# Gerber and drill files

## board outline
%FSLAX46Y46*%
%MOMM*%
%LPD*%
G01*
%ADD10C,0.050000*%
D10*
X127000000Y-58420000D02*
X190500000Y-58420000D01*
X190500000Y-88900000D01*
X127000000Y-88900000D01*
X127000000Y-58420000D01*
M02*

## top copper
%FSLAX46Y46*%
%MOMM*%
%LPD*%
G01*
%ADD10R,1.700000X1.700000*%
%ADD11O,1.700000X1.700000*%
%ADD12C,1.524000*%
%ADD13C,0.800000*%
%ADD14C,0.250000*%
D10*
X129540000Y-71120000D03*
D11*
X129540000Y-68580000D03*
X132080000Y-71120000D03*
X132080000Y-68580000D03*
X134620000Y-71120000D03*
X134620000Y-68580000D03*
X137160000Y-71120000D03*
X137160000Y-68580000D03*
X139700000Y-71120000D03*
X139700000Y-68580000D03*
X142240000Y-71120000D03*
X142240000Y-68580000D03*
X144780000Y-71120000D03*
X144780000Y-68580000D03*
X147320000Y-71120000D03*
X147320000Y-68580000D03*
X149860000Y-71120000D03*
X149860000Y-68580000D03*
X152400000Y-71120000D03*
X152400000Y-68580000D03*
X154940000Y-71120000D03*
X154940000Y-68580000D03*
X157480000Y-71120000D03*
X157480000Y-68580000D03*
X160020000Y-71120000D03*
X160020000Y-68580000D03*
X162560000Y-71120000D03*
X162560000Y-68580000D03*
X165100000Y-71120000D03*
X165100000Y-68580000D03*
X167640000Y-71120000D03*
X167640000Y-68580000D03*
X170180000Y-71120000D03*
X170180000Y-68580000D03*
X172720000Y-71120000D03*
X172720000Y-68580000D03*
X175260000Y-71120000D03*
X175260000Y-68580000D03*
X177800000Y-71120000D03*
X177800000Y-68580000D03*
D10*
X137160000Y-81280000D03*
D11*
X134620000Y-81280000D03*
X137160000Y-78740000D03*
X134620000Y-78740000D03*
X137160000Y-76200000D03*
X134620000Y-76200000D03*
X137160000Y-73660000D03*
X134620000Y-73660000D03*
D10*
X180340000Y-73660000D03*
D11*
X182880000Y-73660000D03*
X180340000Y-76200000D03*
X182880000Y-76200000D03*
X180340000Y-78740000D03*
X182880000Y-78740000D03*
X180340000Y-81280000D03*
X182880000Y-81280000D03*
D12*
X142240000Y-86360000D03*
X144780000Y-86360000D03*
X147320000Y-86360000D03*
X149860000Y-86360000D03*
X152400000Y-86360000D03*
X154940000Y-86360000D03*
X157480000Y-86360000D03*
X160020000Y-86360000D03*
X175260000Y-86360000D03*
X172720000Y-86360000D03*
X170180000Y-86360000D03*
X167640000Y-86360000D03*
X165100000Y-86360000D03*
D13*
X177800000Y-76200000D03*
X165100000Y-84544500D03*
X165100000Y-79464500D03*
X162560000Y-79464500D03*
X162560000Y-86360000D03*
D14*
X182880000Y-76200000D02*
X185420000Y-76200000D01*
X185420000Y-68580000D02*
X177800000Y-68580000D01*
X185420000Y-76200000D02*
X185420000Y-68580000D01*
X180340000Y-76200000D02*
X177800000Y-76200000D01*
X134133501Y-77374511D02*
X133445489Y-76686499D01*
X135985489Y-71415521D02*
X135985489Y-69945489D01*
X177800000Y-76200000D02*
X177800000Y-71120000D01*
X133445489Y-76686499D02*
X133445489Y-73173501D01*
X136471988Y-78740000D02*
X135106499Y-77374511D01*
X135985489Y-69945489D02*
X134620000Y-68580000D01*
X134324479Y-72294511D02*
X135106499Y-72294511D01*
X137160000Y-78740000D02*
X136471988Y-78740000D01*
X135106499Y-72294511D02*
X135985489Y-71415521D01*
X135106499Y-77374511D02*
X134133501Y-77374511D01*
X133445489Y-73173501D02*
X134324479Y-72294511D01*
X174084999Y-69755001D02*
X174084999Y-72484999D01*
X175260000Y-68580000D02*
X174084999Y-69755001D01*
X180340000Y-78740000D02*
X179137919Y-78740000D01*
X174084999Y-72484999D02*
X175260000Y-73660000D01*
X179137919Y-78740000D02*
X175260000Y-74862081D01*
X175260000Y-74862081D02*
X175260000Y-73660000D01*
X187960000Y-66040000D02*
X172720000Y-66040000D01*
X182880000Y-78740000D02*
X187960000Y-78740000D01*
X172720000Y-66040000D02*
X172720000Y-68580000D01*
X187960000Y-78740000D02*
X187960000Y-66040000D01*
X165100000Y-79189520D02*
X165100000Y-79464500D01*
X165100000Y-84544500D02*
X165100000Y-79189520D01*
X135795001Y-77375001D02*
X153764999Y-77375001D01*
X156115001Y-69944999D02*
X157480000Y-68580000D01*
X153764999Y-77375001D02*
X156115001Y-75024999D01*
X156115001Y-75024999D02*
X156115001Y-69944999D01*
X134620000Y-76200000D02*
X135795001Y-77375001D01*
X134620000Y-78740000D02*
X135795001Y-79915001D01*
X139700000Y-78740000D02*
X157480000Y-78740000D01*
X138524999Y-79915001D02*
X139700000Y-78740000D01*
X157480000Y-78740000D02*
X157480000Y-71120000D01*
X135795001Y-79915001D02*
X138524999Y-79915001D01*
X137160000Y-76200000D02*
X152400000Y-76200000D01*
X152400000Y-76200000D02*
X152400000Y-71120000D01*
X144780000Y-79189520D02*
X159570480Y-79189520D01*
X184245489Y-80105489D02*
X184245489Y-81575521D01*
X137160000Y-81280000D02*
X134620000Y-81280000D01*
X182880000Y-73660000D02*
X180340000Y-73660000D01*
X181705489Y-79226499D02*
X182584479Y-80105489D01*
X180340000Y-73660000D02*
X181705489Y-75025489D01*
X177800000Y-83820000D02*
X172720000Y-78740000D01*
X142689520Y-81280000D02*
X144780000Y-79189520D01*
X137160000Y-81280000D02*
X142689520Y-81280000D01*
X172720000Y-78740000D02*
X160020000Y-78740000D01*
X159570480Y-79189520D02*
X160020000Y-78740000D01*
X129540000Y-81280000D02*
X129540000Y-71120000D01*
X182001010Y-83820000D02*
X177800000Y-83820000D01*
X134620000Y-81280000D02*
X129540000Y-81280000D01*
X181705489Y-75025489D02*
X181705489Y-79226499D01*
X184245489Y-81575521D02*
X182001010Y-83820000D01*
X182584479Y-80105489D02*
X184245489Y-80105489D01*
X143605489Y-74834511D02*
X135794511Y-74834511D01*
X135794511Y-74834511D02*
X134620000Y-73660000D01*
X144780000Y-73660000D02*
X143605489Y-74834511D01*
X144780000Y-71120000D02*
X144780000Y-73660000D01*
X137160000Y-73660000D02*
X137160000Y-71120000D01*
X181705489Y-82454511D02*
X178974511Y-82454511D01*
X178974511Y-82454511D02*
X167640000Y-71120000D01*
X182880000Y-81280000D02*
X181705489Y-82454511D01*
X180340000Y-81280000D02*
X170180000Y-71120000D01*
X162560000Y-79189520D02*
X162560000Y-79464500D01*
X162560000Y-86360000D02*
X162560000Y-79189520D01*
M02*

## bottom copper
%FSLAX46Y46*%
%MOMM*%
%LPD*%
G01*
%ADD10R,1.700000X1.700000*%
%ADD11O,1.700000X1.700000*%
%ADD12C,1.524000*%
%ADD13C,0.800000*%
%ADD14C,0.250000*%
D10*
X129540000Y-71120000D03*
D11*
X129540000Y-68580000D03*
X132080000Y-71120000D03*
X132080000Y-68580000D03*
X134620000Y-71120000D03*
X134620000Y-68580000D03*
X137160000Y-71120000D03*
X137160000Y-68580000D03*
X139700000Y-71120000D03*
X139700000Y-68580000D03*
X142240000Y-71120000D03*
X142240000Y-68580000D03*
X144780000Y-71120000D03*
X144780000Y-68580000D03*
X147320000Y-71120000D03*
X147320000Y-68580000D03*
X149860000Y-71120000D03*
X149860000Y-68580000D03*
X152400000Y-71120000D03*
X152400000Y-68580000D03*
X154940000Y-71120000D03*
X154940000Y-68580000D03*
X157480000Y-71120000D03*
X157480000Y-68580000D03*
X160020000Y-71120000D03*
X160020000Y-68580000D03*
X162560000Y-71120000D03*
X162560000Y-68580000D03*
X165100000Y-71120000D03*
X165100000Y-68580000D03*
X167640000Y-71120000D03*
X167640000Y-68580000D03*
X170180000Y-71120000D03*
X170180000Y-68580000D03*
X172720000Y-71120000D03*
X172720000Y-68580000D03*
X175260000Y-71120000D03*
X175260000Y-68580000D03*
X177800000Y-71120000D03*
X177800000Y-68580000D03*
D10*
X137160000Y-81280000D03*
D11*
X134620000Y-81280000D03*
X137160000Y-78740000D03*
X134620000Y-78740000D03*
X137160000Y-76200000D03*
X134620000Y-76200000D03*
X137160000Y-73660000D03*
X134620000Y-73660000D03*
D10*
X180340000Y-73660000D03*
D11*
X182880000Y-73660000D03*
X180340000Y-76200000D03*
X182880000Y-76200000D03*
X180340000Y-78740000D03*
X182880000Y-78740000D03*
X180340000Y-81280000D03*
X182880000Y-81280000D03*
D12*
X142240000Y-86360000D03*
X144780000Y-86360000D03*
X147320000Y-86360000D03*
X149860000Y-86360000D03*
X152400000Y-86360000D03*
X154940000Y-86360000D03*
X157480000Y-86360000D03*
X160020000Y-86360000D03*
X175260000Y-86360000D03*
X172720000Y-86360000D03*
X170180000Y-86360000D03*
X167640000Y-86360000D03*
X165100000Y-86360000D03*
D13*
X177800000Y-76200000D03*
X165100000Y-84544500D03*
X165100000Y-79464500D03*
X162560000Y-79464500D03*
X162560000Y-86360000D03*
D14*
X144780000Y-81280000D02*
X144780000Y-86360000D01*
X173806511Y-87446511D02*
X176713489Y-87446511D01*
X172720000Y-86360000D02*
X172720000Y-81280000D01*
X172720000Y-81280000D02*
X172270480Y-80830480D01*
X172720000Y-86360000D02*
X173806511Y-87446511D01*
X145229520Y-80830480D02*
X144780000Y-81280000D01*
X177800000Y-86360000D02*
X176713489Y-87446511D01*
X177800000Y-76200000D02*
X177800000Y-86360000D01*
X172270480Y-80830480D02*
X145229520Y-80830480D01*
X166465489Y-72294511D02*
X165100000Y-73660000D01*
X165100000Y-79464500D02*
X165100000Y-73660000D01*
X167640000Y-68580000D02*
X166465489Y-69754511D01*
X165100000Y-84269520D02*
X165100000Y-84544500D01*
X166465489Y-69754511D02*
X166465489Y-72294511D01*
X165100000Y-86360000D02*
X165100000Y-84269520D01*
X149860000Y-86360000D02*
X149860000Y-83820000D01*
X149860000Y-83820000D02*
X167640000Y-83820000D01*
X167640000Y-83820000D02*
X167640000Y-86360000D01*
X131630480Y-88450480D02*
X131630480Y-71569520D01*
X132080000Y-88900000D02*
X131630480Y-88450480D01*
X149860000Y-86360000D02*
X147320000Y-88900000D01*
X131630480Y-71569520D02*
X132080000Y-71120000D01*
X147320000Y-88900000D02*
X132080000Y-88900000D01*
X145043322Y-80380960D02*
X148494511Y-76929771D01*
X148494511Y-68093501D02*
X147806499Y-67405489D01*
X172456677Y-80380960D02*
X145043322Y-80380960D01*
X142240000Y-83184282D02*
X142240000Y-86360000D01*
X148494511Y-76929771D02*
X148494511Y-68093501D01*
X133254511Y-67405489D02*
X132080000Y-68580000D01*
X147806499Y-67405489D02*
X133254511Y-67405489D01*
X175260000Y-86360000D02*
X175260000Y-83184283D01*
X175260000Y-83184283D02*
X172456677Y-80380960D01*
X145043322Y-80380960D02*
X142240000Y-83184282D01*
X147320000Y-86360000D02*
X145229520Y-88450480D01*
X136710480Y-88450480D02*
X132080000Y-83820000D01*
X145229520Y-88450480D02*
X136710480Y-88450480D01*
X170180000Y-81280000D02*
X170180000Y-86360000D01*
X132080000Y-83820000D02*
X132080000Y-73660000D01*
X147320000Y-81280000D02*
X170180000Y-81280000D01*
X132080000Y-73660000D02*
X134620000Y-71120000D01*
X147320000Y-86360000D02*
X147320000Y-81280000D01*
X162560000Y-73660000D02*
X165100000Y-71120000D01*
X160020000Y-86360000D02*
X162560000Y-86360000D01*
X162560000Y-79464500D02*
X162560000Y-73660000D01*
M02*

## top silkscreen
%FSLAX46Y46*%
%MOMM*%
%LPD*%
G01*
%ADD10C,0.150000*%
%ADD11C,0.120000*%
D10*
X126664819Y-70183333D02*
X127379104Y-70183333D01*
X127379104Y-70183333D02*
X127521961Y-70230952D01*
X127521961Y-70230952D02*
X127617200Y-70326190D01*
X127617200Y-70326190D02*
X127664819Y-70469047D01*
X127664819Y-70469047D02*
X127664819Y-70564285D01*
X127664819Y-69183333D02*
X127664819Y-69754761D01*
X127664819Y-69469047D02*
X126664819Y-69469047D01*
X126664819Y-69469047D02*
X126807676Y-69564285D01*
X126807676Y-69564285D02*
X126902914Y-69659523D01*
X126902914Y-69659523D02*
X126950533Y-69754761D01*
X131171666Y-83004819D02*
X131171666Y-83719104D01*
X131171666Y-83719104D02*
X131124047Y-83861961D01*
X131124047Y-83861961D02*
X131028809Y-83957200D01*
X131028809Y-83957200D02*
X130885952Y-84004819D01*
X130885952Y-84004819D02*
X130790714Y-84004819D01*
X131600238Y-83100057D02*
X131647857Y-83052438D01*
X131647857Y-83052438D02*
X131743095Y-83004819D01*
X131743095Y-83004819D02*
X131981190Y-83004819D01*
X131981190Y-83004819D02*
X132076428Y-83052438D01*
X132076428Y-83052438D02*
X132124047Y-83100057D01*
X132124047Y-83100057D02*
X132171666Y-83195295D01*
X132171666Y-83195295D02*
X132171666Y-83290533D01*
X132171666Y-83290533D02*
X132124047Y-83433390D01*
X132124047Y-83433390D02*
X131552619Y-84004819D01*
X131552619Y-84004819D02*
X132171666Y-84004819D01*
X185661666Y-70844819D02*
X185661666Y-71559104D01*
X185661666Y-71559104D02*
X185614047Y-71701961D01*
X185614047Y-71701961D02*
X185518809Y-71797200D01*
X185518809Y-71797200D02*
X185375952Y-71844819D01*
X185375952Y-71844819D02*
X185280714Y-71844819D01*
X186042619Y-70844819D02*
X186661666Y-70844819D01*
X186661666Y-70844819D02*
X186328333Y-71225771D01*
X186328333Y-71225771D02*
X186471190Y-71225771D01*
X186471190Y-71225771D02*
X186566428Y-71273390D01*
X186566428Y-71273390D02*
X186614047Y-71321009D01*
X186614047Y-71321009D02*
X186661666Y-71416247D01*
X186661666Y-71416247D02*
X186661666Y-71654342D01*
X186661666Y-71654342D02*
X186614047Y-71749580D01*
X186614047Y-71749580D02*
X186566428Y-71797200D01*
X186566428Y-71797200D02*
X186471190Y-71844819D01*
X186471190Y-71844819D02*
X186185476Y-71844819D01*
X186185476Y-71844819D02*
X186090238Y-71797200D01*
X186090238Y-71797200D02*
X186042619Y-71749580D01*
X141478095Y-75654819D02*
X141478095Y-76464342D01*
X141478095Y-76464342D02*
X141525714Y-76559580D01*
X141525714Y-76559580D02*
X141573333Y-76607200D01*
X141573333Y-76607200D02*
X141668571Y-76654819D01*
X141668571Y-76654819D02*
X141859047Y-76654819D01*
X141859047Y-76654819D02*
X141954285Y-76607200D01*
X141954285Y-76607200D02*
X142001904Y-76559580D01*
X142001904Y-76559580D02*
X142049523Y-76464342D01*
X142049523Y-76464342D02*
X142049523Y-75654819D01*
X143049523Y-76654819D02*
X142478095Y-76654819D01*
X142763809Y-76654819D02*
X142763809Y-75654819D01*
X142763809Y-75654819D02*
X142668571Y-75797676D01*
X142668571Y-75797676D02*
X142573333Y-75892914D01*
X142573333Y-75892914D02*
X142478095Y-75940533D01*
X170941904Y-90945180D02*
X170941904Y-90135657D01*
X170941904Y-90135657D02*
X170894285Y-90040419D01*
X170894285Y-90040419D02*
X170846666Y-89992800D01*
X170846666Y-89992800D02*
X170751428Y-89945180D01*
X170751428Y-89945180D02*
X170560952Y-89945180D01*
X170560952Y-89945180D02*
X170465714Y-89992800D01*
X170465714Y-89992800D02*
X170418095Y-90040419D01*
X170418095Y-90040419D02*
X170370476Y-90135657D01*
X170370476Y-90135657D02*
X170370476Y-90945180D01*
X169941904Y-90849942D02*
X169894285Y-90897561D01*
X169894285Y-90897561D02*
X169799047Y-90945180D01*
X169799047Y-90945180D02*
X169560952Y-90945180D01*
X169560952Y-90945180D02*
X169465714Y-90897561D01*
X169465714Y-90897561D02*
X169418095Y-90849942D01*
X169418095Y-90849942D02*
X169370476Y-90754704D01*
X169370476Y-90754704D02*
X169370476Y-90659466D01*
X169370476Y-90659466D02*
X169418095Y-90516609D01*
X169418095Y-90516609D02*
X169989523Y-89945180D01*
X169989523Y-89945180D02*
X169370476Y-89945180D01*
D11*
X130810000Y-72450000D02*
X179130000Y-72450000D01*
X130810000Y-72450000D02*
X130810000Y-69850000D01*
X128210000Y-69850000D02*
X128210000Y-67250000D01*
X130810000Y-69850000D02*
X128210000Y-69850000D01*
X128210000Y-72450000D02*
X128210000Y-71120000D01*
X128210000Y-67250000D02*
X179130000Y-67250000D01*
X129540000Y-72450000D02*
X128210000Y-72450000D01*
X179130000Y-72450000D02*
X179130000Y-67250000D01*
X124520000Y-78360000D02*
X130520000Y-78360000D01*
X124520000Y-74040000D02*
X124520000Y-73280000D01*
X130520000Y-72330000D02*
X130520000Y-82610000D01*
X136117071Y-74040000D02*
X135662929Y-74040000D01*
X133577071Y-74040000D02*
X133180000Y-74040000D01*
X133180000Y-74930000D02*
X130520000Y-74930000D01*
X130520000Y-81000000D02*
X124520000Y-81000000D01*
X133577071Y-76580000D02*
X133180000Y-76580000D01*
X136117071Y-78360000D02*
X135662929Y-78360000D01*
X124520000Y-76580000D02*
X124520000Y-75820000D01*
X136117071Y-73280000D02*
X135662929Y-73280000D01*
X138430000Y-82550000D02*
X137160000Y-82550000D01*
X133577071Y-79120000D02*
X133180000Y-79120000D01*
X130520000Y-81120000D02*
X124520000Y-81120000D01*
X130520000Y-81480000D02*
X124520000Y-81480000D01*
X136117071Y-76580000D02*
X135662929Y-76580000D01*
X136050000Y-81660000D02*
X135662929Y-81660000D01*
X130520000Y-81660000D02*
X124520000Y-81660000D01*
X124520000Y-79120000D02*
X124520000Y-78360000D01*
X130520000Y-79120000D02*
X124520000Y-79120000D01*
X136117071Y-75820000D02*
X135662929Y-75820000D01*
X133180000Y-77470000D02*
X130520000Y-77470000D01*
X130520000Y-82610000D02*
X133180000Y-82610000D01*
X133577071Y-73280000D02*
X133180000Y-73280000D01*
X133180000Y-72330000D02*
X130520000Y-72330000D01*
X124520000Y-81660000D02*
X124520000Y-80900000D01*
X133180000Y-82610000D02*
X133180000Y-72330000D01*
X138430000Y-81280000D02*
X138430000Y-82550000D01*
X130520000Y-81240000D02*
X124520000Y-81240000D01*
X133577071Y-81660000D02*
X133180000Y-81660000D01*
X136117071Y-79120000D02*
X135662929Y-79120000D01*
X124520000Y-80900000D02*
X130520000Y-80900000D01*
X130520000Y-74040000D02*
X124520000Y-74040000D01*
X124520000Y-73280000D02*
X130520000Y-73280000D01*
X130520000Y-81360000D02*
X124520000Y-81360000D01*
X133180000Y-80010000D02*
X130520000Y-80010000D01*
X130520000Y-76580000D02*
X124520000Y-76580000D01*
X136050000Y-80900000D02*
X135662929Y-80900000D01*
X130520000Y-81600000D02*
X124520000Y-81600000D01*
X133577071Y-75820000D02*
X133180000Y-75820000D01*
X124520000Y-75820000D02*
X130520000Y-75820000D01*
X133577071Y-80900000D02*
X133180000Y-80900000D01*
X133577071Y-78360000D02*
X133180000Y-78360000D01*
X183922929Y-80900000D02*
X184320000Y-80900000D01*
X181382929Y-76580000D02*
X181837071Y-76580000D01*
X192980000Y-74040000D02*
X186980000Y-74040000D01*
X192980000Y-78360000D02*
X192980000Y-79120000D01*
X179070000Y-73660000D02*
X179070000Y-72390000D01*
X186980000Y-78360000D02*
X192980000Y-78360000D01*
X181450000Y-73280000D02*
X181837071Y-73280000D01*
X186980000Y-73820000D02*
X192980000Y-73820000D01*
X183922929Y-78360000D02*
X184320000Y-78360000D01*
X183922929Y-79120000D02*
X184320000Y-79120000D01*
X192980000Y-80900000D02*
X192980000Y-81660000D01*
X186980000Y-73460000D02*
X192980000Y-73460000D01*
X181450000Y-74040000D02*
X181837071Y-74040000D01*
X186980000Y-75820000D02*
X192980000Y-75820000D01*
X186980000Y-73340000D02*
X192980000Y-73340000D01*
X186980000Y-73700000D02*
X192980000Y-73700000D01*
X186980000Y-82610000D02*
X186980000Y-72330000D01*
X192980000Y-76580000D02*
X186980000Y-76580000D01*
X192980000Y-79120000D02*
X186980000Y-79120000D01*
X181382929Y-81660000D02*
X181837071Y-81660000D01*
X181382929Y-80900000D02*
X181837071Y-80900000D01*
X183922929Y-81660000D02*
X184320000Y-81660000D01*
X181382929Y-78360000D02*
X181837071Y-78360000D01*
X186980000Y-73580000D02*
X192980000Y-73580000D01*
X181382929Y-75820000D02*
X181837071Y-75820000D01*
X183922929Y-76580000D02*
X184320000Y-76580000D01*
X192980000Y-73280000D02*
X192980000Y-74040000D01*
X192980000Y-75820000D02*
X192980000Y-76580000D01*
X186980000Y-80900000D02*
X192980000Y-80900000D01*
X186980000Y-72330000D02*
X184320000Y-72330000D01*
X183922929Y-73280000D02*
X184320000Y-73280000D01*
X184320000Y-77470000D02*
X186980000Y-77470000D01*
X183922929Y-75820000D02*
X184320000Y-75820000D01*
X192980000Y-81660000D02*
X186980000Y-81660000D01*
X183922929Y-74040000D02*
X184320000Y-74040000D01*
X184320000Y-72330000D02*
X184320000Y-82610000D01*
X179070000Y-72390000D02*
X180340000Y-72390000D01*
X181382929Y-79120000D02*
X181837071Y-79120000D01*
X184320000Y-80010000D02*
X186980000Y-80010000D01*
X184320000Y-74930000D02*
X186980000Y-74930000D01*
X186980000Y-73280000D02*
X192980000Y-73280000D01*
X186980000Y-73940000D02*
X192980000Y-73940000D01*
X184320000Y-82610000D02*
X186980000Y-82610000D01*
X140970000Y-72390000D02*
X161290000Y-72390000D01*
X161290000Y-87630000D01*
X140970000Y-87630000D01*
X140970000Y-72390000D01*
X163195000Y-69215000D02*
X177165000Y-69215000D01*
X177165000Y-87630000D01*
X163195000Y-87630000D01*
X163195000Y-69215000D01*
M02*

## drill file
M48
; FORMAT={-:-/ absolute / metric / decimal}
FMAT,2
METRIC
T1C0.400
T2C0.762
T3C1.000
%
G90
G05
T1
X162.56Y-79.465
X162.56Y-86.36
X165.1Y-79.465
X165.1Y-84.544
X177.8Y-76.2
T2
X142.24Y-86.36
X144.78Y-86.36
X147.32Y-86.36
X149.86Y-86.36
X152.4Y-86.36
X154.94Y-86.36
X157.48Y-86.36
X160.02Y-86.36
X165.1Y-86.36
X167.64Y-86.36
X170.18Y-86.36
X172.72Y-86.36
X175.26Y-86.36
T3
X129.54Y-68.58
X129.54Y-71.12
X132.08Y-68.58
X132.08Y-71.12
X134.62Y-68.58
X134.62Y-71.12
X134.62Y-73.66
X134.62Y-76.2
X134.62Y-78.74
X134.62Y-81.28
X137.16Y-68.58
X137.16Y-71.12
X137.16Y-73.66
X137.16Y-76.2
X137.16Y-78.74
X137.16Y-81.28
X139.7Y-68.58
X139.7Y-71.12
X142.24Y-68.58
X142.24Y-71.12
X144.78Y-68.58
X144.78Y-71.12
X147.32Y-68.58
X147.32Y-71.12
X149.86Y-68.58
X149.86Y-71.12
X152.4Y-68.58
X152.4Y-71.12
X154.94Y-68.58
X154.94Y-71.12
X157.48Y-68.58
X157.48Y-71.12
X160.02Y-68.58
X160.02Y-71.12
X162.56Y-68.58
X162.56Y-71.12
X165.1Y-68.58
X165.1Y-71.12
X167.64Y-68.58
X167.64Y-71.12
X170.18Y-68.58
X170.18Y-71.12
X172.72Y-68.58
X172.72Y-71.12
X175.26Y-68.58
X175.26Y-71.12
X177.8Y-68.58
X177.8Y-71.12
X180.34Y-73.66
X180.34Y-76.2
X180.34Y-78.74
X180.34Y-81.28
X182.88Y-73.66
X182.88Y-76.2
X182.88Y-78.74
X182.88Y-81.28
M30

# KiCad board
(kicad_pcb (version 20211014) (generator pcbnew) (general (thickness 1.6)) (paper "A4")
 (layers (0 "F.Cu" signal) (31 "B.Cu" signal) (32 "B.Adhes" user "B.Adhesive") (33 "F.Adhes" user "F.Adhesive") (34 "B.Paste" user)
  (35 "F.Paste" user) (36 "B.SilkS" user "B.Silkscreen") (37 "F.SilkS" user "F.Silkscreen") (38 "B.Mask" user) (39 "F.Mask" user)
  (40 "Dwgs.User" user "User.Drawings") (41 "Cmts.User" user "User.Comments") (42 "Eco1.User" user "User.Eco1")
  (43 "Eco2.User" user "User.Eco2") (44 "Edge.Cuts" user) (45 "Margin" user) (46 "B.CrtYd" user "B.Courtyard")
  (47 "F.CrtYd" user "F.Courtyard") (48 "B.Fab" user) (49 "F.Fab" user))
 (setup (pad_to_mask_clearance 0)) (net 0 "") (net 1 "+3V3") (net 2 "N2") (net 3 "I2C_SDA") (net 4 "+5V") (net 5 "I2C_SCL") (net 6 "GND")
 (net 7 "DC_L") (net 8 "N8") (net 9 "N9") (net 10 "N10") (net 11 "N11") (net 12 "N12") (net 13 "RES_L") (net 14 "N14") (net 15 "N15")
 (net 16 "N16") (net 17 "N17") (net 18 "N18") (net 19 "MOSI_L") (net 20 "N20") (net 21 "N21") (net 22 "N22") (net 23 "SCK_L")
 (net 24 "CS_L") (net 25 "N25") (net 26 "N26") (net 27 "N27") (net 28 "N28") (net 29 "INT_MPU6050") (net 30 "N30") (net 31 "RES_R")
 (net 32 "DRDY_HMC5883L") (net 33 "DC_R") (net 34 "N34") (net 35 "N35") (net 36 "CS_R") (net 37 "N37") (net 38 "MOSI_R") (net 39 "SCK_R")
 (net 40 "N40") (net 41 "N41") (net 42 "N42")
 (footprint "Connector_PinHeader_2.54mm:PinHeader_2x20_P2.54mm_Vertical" (layer "F.Cu") (at 129.54 71.12 90)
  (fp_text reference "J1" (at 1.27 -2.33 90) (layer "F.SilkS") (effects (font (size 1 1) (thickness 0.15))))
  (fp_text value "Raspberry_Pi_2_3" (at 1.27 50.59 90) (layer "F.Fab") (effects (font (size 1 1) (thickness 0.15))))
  (fp_line (start -1.33 1.27) (end -1.33 49.59) (layer "F.SilkS") (width 0.12))
  (fp_line (start -1.33 1.27) (end 1.27 1.27) (layer "F.SilkS") (width 0.12))
  (fp_line (start 1.27 -1.33) (end 3.87 -1.33) (layer "F.SilkS") (width 0.12))
  (fp_line (start 1.27 1.27) (end 1.27 -1.33) (layer "F.SilkS") (width 0.12))
  (fp_line (start -1.33 -1.33) (end 0 -1.33) (layer "F.SilkS") (width 0.12))
  (fp_line (start 3.87 -1.33) (end 3.87 49.59) (layer "F.SilkS") (width 0.12))
  (fp_line (start -1.33 0) (end -1.33 -1.33) (layer "F.SilkS") (width 0.12))
  (fp_line (start -1.33 49.59) (end 3.87 49.59) (layer "F.SilkS") (width 0.12))
  (pad "1" thru_hole rect locked (at 0 0 90) (size 1.7 1.7) (drill 1) (layers *.Cu *.Mask) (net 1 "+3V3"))
  (pad "2" thru_hole oval locked (at 2.54 0 90) (size 1.7 1.7) (drill 1) (layers *.Cu *.Mask) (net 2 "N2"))
  (pad "3" thru_hole oval locked (at 0 2.54 90) (size 1.7 1.7) (drill 1) (layers *.Cu *.Mask) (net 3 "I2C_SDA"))
  (pad "4" thru_hole oval locked (at 2.54 2.54 90) (size 1.7 1.7) (drill 1) (layers *.Cu *.Mask) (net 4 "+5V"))
  (pad "5" thru_hole oval locked (at 0 5.08 90) (size 1.7 1.7) (drill 1) (layers *.Cu *.Mask) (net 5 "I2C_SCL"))
  (pad "6" thru_hole oval locked (at 2.54 5.08 90) (size 1.7 1.7) (drill 1) (layers *.Cu *.Mask) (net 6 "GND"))
  (pad "7" thru_hole oval locked (at 0 7.62 90) (size 1.7 1.7) (drill 1) (layers *.Cu *.Mask) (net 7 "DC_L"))
  (pad "8" thru_hole oval locked (at 2.54 7.62 90) (size 1.7 1.7) (drill 1) (layers *.Cu *.Mask) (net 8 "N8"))
  (pad "9" thru_hole oval locked (at 0 10.16 90) (size 1.7 1.7) (drill 1) (layers *.Cu *.Mask) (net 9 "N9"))
  (pad "10" thru_hole oval locked (at 2.54 10.16 90) (size 1.7 1.7) (drill 1) (layers *.Cu *.Mask) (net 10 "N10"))
  (pad "11" thru_hole oval locked (at 0 12.7 90) (size 1.7 1.7) (drill 1) (layers *.Cu *.Mask) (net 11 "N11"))
  (pad "12" thru_hole oval locked (at 2.54 12.7 90) (size 1.7 1.7) (drill 1) (layers *.Cu *.Mask) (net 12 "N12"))
  (pad "13" thru_hole oval locked (at 0 15.24 90) (size 1.7 1.7) (drill 1) (layers *.Cu *.Mask) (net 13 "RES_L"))
  (pad "14" thru_hole oval locked (at 2.54 15.24 90) (size 1.7 1.7) (drill 1) (layers *.Cu *.Mask) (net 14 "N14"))
  (pad "15" thru_hole oval locked (at 0 17.78 90) (size 1.7 1.7) (drill 1) (layers *.Cu *.Mask) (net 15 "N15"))
  (pad "16" thru_hole oval locked (at 2.54 17.78 90) (size 1.7 1.7) (drill 1) (layers *.Cu *.Mask) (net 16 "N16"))
  (pad "17" thru_hole oval locked (at 0 20.32 90) (size 1.7 1.7) (drill 1) (layers *.Cu *.Mask) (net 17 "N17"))
  (pad "18" thru_hole oval locked (at 2.54 20.32 90) (size 1.7 1.7) (drill 1) (layers *.Cu *.Mask) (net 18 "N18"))
  (pad "19" thru_hole oval locked (at 0 22.86 90) (size 1.7 1.7) (drill 1) (layers *.Cu *.Mask) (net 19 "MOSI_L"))
  (pad "20" thru_hole oval locked (at 2.54 22.86 90) (size 1.7 1.7) (drill 1) (layers *.Cu *.Mask) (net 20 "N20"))
  (pad "21" thru_hole oval locked (at 0 25.4 90) (size 1.7 1.7) (drill 1) (layers *.Cu *.Mask) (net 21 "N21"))
  (pad "22" thru_hole oval locked (at 2.54 25.4 90) (size 1.7 1.7) (drill 1) (layers *.Cu *.Mask) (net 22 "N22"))
  (pad "23" thru_hole oval locked (at 0 27.94 90) (size 1.7 1.7) (drill 1) (layers *.Cu *.Mask) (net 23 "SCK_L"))
  (pad "24" thru_hole oval locked (at 2.54 27.94 90) (size 1.7 1.7) (drill 1) (layers *.Cu *.Mask) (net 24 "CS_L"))
  (pad "25" thru_hole oval locked (at 0 30.48 90) (size 1.7 1.7) (drill 1) (layers *.Cu *.Mask) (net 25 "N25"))
  (pad "26" thru_hole oval locked (at 2.54 30.48 90) (size 1.7 1.7) (drill 1) (layers *.Cu *.Mask) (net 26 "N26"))
  (pad "27" thru_hole oval locked (at 0 33.02 90) (size 1.7 1.7) (drill 1) (layers *.Cu *.Mask) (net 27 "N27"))
  (pad "28" thru_hole oval locked (at 2.54 33.02 90) (size 1.7 1.7) (drill 1) (layers *.Cu *.Mask) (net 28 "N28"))
  (pad "29" thru_hole oval locked (at 0 35.56 90) (size 1.7 1.7) (drill 1) (layers *.Cu *.Mask) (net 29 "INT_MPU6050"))
  (pad "30" thru_hole oval locked (at 2.54 35.56 90) (size 1.7 1.7) (drill 1) (layers *.Cu *.Mask) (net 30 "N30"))
  (pad "31" thru_hole oval locked (at 0 38.1 90) (size 1.7 1.7) (drill 1) (layers *.Cu *.Mask) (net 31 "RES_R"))
  (pad "32" thru_hole oval locked (at 2.54 38.1 90) (size 1.7 1.7) (drill 1) (layers *.Cu *.Mask) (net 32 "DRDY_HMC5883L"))
  (pad "33" thru_hole oval locked (at 0 40.64 90) (size 1.7 1.7) (drill 1) (layers *.Cu *.Mask) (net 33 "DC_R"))
  (pad "34" thru_hole oval locked (at 2.54 40.64 90) (size 1.7 1.7) (drill 1) (layers *.Cu *.Mask) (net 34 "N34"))
  (pad "35" thru_hole oval locked (at 0 43.18 90) (size 1.7 1.7) (drill 1) (layers *.Cu *.Mask) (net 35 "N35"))
  (pad "36" thru_hole oval locked (at 2.54 43.18 90) (size 1.7 1.7) (drill 1) (layers *.Cu *.Mask) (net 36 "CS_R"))
  (pad "37" thru_hole oval locked (at 0 45.72 90) (size 1.7 1.7) (drill 1) (layers *.Cu *.Mask) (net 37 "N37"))
  (pad "38" thru_hole oval locked (at 2.54 45.72 90) (size 1.7 1.7) (drill 1) (layers *.Cu *.Mask) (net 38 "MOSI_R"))
  (pad "39" thru_hole oval locked (at 0 48.26 90) (size 1.7 1.7) (drill 1) (layers *.Cu *.Mask) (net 6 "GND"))
  (pad "40" thru_hole oval locked (at 2.54 48.26 90) (size 1.7 1.7) (drill 1) (layers *.Cu *.Mask) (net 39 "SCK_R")))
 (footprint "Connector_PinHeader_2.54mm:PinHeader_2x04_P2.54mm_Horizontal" (layer "F.Cu") (at 137.16 81.28 180)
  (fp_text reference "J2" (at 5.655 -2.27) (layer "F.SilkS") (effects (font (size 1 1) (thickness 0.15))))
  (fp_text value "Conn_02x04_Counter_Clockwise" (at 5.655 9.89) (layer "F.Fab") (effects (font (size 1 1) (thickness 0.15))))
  (fp_line (start 12.64 2.92) (end 6.64 2.92) (layer "F.SilkS") (width 0.12))
  (fp_line (start 12.64 7.24) (end 12.64 8) (layer "F.SilkS") (width 0.12))
  (fp_line (start 6.64 8.95) (end 6.64 -1.33) (layer "F.SilkS") (width 0.12))
  (fp_line (start 1.042929 7.24) (end 1.497071 7.24) (layer "F.SilkS") (width 0.12))
  (fp_line (start 3.582929 7.24) (end 3.98 7.24) (layer "F.SilkS") (width 0.12))
  (fp_line (start 3.98 6.35) (end 6.64 6.35) (layer "F.SilkS") (width 0.12))
  (fp_line (start 6.64 0.28) (end 12.64 0.28) (layer "F.SilkS") (width 0.12))
  (fp_line (start 3.582929 4.7) (end 3.98 4.7) (layer "F.SilkS") (width 0.12))
  (fp_line (start 1.042929 2.92) (end 1.497071 2.92) (layer "F.SilkS") (width 0.12))
  (fp_line (start 12.64 4.7) (end 12.64 5.46) (layer "F.SilkS") (width 0.12))
  (fp_line (start 1.042929 8) (end 1.497071 8) (layer "F.SilkS") (width 0.12))
  (fp_line (start -1.27 -1.27) (end 0 -1.27) (layer "F.SilkS") (width 0.12))
  (fp_line (start 3.582929 2.16) (end 3.98 2.16) (layer "F.SilkS") (width 0.12))
  (fp_line (start 6.64 0.16) (end 12.64 0.16) (layer "F.SilkS") (width 0.12))
  (fp_line (start 6.64 -0.2) (end 12.64 -0.2) (layer "F.SilkS") (width 0.12))
  (fp_line (start 1.042929 4.7) (end 1.497071 4.7) (layer "F.SilkS") (width 0.12))
  (fp_line (start 1.11 -0.38) (end 1.497071 -0.38) (layer "F.SilkS") (width 0.12))
  (fp_line (start 6.64 -0.38) (end 12.64 -0.38) (layer "F.SilkS") (width 0.12))
  (fp_line (start 12.64 2.16) (end 12.64 2.92) (layer "F.SilkS") (width 0.12))
  (fp_line (start 6.64 2.16) (end 12.64 2.16) (layer "F.SilkS") (width 0.12))
  (fp_line (start 1.042929 5.46) (end 1.497071 5.46) (layer "F.SilkS") (width 0.12))
  (fp_line (start 3.98 3.81) (end 6.64 3.81) (layer "F.SilkS") (width 0.12))
  (fp_line (start 6.64 -1.33) (end 3.98 -1.33) (layer "F.SilkS") (width 0.12))
  (fp_line (start 3.582929 8) (end 3.98 8) (layer "F.SilkS") (width 0.12))
  (fp_line (start 3.98 8.95) (end 6.64 8.95) (layer "F.SilkS") (width 0.12))
  (fp_line (start 12.64 -0.38) (end 12.64 0.38) (layer "F.SilkS") (width 0.12))
  (fp_line (start 3.98 -1.33) (end 3.98 8.95) (layer "F.SilkS") (width 0.12))
  (fp_line (start -1.27 0) (end -1.27 -1.27) (layer "F.SilkS") (width 0.12))
  (fp_line (start 6.64 0.04) (end 12.64 0.04) (layer "F.SilkS") (width 0.12))
  (fp_line (start 3.582929 -0.38) (end 3.98 -0.38) (layer "F.SilkS") (width 0.12))
  (fp_line (start 1.042929 2.16) (end 1.497071 2.16) (layer "F.SilkS") (width 0.12))
  (fp_line (start 12.64 0.38) (end 6.64 0.38) (layer "F.SilkS") (width 0.12))
  (fp_line (start 6.64 7.24) (end 12.64 7.24) (layer "F.SilkS") (width 0.12))
  (fp_line (start 12.64 8) (end 6.64 8) (layer "F.SilkS") (width 0.12))
  (fp_line (start 6.64 -0.08) (end 12.64 -0.08) (layer "F.SilkS") (width 0.12))
  (fp_line (start 3.98 1.27) (end 6.64 1.27) (layer "F.SilkS") (width 0.12))
  (fp_line (start 6.64 4.7) (end 12.64 4.7) (layer "F.SilkS") (width 0.12))
  (fp_line (start 1.11 0.38) (end 1.497071 0.38) (layer "F.SilkS") (width 0.12))
  (fp_line (start 6.64 -0.32) (end 12.64 -0.32) (layer "F.SilkS") (width 0.12))
  (fp_line (start 3.582929 5.46) (end 3.98 5.46) (layer "F.SilkS") (width 0.12))
  (fp_line (start 12.64 5.46) (end 6.64 5.46) (layer "F.SilkS") (width 0.12))
  (fp_line (start 3.582929 0.38) (end 3.98 0.38) (layer "F.SilkS") (width 0.12))
  (fp_line (start 3.582929 2.92) (end 3.98 2.92) (layer "F.SilkS") (width 0.12))
  (pad "1" thru_hole rect locked (at 0 0 180) (size 1.7 1.7) (drill 1) (layers *.Cu *.Mask) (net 1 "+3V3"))
  (pad "2" thru_hole oval locked (at 2.54 0 180) (size 1.7 1.7) (drill 1) (layers *.Cu *.Mask) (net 1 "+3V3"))
  (pad "3" thru_hole oval locked (at 0 2.54 180) (size 1.7 1.7) (drill 1) (layers *.Cu *.Mask) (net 6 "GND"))
  (pad "4" thru_hole oval locked (at 2.54 2.54 180) (size 1.7 1.7) (drill 1) (layers *.Cu *.Mask) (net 23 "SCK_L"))
  (pad "5" thru_hole oval locked (at 0 5.08 180) (size 1.7 1.7) (drill 1) (layers *.Cu *.Mask) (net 19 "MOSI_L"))
  (pad "6" thru_hole oval locked (at 2.54 5.08 180) (size 1.7 1.7) (drill 1) (layers *.Cu *.Mask) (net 24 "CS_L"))
  (pad "7" thru_hole oval locked (at 0 7.62 180) (size 1.7 1.7) (drill 1) (layers *.Cu *.Mask) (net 7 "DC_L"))
  (pad "8" thru_hole oval locked (at 2.54 7.62 180) (size 1.7 1.7) (drill 1) (layers *.Cu *.Mask) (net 13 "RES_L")))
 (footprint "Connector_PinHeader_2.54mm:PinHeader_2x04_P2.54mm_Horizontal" (layer "F.Cu") (at 180.34 73.66)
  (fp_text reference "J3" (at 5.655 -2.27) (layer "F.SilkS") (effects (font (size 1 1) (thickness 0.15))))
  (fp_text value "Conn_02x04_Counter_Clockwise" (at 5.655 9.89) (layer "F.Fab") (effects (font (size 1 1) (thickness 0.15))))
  (fp_line (start 3.582929 7.24) (end 3.98 7.24) (layer "F.SilkS") (width 0.12))
  (fp_line (start 1.042929 2.92) (end 1.497071 2.92) (layer "F.SilkS") (width 0.12))
  (fp_line (start 12.64 0.38) (end 6.64 0.38) (layer "F.SilkS") (width 0.12))
  (fp_line (start 12.64 4.7) (end 12.64 5.46) (layer "F.SilkS") (width 0.12))
  (fp_line (start -1.27 0) (end -1.27 -1.27) (layer "F.SilkS") (width 0.12))
  (fp_line (start 6.64 4.7) (end 12.64 4.7) (layer "F.SilkS") (width 0.12))
  (fp_line (start 1.11 -0.38) (end 1.497071 -0.38) (layer "F.SilkS") (width 0.12))
  (fp_line (start 6.64 0.16) (end 12.64 0.16) (layer "F.SilkS") (width 0.12))
  (fp_line (start 3.582929 4.7) (end 3.98 4.7) (layer "F.SilkS") (width 0.12))
  (fp_line (start 3.582929 5.46) (end 3.98 5.46) (layer "F.SilkS") (width 0.12))
  (fp_line (start 12.64 7.24) (end 12.64 8) (layer "F.SilkS") (width 0.12))
  (fp_line (start 6.64 -0.2) (end 12.64 -0.2) (layer "F.SilkS") (width 0.12))
  (fp_line (start 1.11 0.38) (end 1.497071 0.38) (layer "F.SilkS") (width 0.12))
  (fp_line (start 6.64 2.16) (end 12.64 2.16) (layer "F.SilkS") (width 0.12))
  (fp_line (start 6.64 -0.32) (end 12.64 -0.32) (layer "F.SilkS") (width 0.12))
  (fp_line (start 6.64 0.04) (end 12.64 0.04) (layer "F.SilkS") (width 0.12))
  (fp_line (start 6.64 8.95) (end 6.64 -1.33) (layer "F.SilkS") (width 0.12))
  (fp_line (start 12.64 2.92) (end 6.64 2.92) (layer "F.SilkS") (width 0.12))
  (fp_line (start 12.64 5.46) (end 6.64 5.46) (layer "F.SilkS") (width 0.12))
  (fp_line (start 1.042929 8) (end 1.497071 8) (layer "F.SilkS") (width 0.12))
  (fp_line (start 1.042929 7.24) (end 1.497071 7.24) (layer "F.SilkS") (width 0.12))
  (fp_line (start 3.582929 8) (end 3.98 8) (layer "F.SilkS") (width 0.12))
  (fp_line (start 1.042929 4.7) (end 1.497071 4.7) (layer "F.SilkS") (width 0.12))
  (fp_line (start 6.64 -0.08) (end 12.64 -0.08) (layer "F.SilkS") (width 0.12))
  (fp_line (start 1.042929 2.16) (end 1.497071 2.16) (layer "F.SilkS") (width 0.12))
  (fp_line (start 3.582929 2.92) (end 3.98 2.92) (layer "F.SilkS") (width 0.12))
  (fp_line (start 12.64 -0.38) (end 12.64 0.38) (layer "F.SilkS") (width 0.12))
  (fp_line (start 12.64 2.16) (end 12.64 2.92) (layer "F.SilkS") (width 0.12))
  (fp_line (start 6.64 7.24) (end 12.64 7.24) (layer "F.SilkS") (width 0.12))
  (fp_line (start 6.64 -1.33) (end 3.98 -1.33) (layer "F.SilkS") (width 0.12))
  (fp_line (start 3.582929 -0.38) (end 3.98 -0.38) (layer "F.SilkS") (width 0.12))
  (fp_line (start 3.98 3.81) (end 6.64 3.81) (layer "F.SilkS") (width 0.12))
  (fp_line (start 3.582929 2.16) (end 3.98 2.16) (layer "F.SilkS") (width 0.12))
  (fp_line (start 12.64 8) (end 6.64 8) (layer "F.SilkS") (width 0.12))
  (fp_line (start 3.582929 0.38) (end 3.98 0.38) (layer "F.SilkS") (width 0.12))
  (fp_line (start 3.98 -1.33) (end 3.98 8.95) (layer "F.SilkS") (width 0.12))
  (fp_line (start -1.27 -1.27) (end 0 -1.27) (layer "F.SilkS") (width 0.12))
  (fp_line (start 1.042929 5.46) (end 1.497071 5.46) (layer "F.SilkS") (width 0.12))
  (fp_line (start 3.98 6.35) (end 6.64 6.35) (layer "F.SilkS") (width 0.12))
  (fp_line (start 3.98 1.27) (end 6.64 1.27) (layer "F.SilkS") (width 0.12))
  (fp_line (start 6.64 -0.38) (end 12.64 -0.38) (layer "F.SilkS") (width 0.12))
  (fp_line (start 6.64 0.28) (end 12.64 0.28) (layer "F.SilkS") (width 0.12))
  (fp_line (start 3.98 8.95) (end 6.64 8.95) (layer "F.SilkS") (width 0.12))
  (pad "1" thru_hole rect locked (at 0 0) (size 1.7 1.7) (drill 1) (layers *.Cu *.Mask) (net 1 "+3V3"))
  (pad "2" thru_hole oval locked (at 2.54 0) (size 1.7 1.7) (drill 1) (layers *.Cu *.Mask) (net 1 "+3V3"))
  (pad "3" thru_hole oval locked (at 0 2.54) (size 1.7 1.7) (drill 1) (layers *.Cu *.Mask) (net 6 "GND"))
  (pad "4" thru_hole oval locked (at 2.54 2.54) (size 1.7 1.7) (drill 1) (layers *.Cu *.Mask) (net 39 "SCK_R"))
  (pad "5" thru_hole oval locked (at 0 5.08) (size 1.7 1.7) (drill 1) (layers *.Cu *.Mask) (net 38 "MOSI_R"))
  (pad "6" thru_hole oval locked (at 2.54 5.08) (size 1.7 1.7) (drill 1) (layers *.Cu *.Mask) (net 36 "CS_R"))
  (pad "7" thru_hole oval locked (at 0 7.62) (size 1.7 1.7) (drill 1) (layers *.Cu *.Mask) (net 33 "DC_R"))
  (pad "8" thru_hole oval locked (at 2.54 7.62) (size 1.7 1.7) (drill 1) (layers *.Cu *.Mask) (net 31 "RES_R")))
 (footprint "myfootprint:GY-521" (layer "F.Cu") (at 142.24 86.36)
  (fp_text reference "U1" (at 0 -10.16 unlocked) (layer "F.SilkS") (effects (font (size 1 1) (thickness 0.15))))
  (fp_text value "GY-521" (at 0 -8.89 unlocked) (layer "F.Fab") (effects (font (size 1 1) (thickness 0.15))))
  (fp_rect (start -1.27 1.27) (end 19.05 -13.97) (layer "F.SilkS") (width 0.12) (fill none))
  (pad "1" thru_hole circle (at 0 0) (size 1.524 1.524) (drill 0.762) (layers *.Cu *.Mask) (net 4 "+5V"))
  (pad "2" thru_hole circle (at 2.54 0) (size 1.524 1.524) (drill 0.762) (layers *.Cu *.Mask) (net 6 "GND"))
  (pad "3" thru_hole circle (at 5.08 0) (size 1.524 1.524) (drill 0.762) (layers *.Cu *.Mask) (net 5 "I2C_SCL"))
  (pad "4" thru_hole circle (at 7.62 0) (size 1.524 1.524) (drill 0.762) (layers *.Cu *.Mask) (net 3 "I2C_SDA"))
  (pad "5" thru_hole circle (at 10.16 0) (size 1.524 1.524) (drill 0.762) (layers *.Cu *.Mask) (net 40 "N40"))
  (pad "6" thru_hole circle (at 12.7 0) (size 1.524 1.524) (drill 0.762) (layers *.Cu *.Mask) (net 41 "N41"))
  (pad "7" thru_hole circle (at 15.24 0) (size 1.524 1.524) (drill 0.762) (layers *.Cu *.Mask) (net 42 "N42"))
  (pad "8" thru_hole circle (at 17.78 0) (size 1.524 1.524) (drill 0.762) (layers *.Cu *.Mask) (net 29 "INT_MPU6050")))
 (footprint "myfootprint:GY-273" (layer "F.Cu") (at 175.26 86.36 180)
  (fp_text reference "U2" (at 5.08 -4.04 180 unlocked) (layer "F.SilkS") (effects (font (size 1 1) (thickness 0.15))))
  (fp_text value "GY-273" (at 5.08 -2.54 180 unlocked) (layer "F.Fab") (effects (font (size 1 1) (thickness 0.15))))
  (fp_rect (start -1.905 -1.27) (end 12.065 17.145) (layer "F.SilkS") (width 0.12) (fill none))
  (pad "1" thru_hole circle (at 0 0 180) (size 1.524 1.524) (drill 0.762) (layers *.Cu *.Mask) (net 4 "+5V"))
  (pad "2" thru_hole circle (at 2.54 0 180) (size 1.524 1.524) (drill 0.762) (layers *.Cu *.Mask) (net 6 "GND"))
  (pad "3" thru_hole circle (at 5.08 0 180) (size 1.524 1.524) (drill 0.762) (layers *.Cu *.Mask) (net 5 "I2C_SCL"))
  (pad "4" thru_hole circle (at 7.62 0 180) (size 1.524 1.524) (drill 0.762) (layers *.Cu *.Mask) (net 3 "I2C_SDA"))
  (pad "5" thru_hole circle (at 10.16 0 180) (size 1.524 1.524) (drill 0.762) (layers *.Cu *.Mask) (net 32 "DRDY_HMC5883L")))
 (gr_rect (start 127 88.9) (end 190.5 58.42) (layer "Edge.Cuts") (width 0.05) (fill none))
 (segment (start 182.88 76.2) (end 185.42 76.2) (width 0.25) (layer "F.Cu") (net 39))
 (segment (start 185.42 68.58) (end 177.8 68.58) (width 0.25) (layer "F.Cu") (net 39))
 (segment (start 185.42 76.2) (end 185.42 68.58) (width 0.25) (layer "F.Cu") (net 39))
 (segment (start 180.34 76.2) (end 177.8 76.2) (width 0.25) (layer "F.Cu") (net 6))
 (segment (start 134.133501 77.374511) (end 133.445489 76.686499) (width 0.25) (layer "F.Cu") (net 6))
 (segment (start 135.985489 71.415521) (end 135.985489 69.945489) (width 0.25) (layer "F.Cu") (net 6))
 (segment (start 177.8 76.2) (end 177.8 71.12) (width 0.25) (layer "F.Cu") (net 6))
 (segment (start 133.445489 76.686499) (end 133.445489 73.173501) (width 0.25) (layer "F.Cu") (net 6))
 (segment (start 136.471988 78.74) (end 135.106499 77.374511) (width 0.25) (layer "F.Cu") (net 6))
 (segment (start 135.985489 69.945489) (end 134.62 68.58) (width 0.25) (layer "F.Cu") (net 6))
 (segment (start 134.324479 72.294511) (end 135.106499 72.294511) (width 0.25) (layer "F.Cu") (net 6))
 (segment (start 137.16 78.74) (end 136.471988 78.74) (width 0.25) (layer "F.Cu") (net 6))
 (segment (start 135.106499 72.294511) (end 135.985489 71.415521) (width 0.25) (layer "F.Cu") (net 6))
 (segment (start 135.106499 77.374511) (end 134.133501 77.374511) (width 0.25) (layer "F.Cu") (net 6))
 (segment (start 133.445489 73.173501) (end 134.324479 72.294511) (width 0.25) (layer "F.Cu") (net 6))
 (via (at 177.8 76.2) (size 0.8) (drill 0.4) (layers "F.Cu" "B.Cu") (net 6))
 (segment (start 144.78 81.28) (end 144.78 86.36) (width 0.25) (layer "B.Cu") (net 6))
 (segment (start 173.806511 87.446511) (end 176.713489 87.446511) (width 0.25) (layer "B.Cu") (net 6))
 (segment (start 172.72 86.36) (end 172.72 81.28) (width 0.25) (layer "B.Cu") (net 6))
 (segment (start 172.72 81.28) (end 172.27048 80.83048) (width 0.25) (layer "B.Cu") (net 6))
 (segment (start 172.72 86.36) (end 173.806511 87.446511) (width 0.25) (layer "B.Cu") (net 6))
 (segment (start 145.22952 80.83048) (end 144.78 81.28) (width 0.25) (layer "B.Cu") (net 6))
 (segment (start 177.8 86.36) (end 176.713489 87.446511) (width 0.25) (layer "B.Cu") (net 6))
 (segment (start 177.8 76.2) (end 177.8 86.36) (width 0.25) (layer "B.Cu") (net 6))
 (segment (start 172.27048 80.83048) (end 145.22952 80.83048) (width 0.25) (layer "B.Cu") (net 6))
 (segment (start 174.084999 69.755001) (end 174.084999 72.484999) (width 0.25) (layer "F.Cu") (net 38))
 (segment (start 175.26 68.58) (end 174.084999 69.755001) (width 0.25) (layer "F.Cu") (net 38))
 (segment (start 180.34 78.74) (end 179.137919 78.74) (width 0.25) (layer "F.Cu") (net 38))
 (segment (start 174.084999 72.484999) (end 175.26 73.66) (width 0.25) (layer "F.Cu") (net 38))
 (segment (start 179.137919 78.74) (end 175.26 74.862081) (width 0.25) (layer "F.Cu") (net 38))
 (segment (start 175.26 74.862081) (end 175.26 73.66) (width 0.25) (layer "F.Cu") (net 38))
 (segment (start 187.96 66.04) (end 172.72 66.04) (width 0.25) (layer "F.Cu") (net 36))
 (segment (start 182.88 78.74) (end 187.96 78.74) (width 0.25) (layer "F.Cu") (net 36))
 (segment (start 172.72 66.04) (end 172.72 68.58) (width 0.25) (layer "F.Cu") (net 36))
 (segment (start 187.96 78.74) (end 187.96 66.04) (width 0.25) (layer "F.Cu") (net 36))
 (segment (start 165.1 79.18952) (end 165.1 79.4645) (width 0.25) (layer "F.Cu") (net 32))
 (segment (start 165.1 84.5445) (end 165.1 79.18952) (width 0.25) (layer "F.Cu") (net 32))
 (via (at 165.1 84.5445) (size 0.8) (drill 0.4) (layers "F.Cu" "B.Cu") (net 32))
 (via (at 165.1 79.4645) (size 0.8) (drill 0.4) (layers "F.Cu" "B.Cu") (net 32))
 (segment (start 166.465489 72.294511) (end 165.1 73.66) (width 0.25) (layer "B.Cu") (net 32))
 (segment (start 165.1 79.4645) (end 165.1 73.66) (width 0.25) (layer "B.Cu") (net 32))
 (segment (start 167.64 68.58) (end 166.465489 69.754511) (width 0.25) (layer "B.Cu") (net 32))
 (segment (start 165.1 84.26952) (end 165.1 84.5445) (width 0.25) (layer "B.Cu") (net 32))
 (segment (start 166.465489 69.754511) (end 166.465489 72.294511) (width 0.25) (layer "B.Cu") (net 32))
 (segment (start 165.1 86.36) (end 165.1 84.26952) (width 0.25) (layer "B.Cu") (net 32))
 (segment (start 135.795001 77.375001) (end 153.764999 77.375001) (width 0.25) (layer "F.Cu") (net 24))
 (segment (start 156.115001 69.944999) (end 157.48 68.58) (width 0.25) (layer "F.Cu") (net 24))
 (segment (start 153.764999 77.375001) (end 156.115001 75.024999) (width 0.25) (layer "F.Cu") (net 24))
 (segment (start 156.115001 75.024999) (end 156.115001 69.944999) (width 0.25) (layer "F.Cu") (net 24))
 (segment (start 134.62 76.2) (end 135.795001 77.375001) (width 0.25) (layer "F.Cu") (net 24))
 (segment (start 134.62 78.74) (end 135.795001 79.915001) (width 0.25) (layer "F.Cu") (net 23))
 (segment (start 139.7 78.74) (end 157.48 78.74) (width 0.25) (layer "F.Cu") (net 23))
 (segment (start 138.524999 79.915001) (end 139.7 78.74) (width 0.25) (layer "F.Cu") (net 23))
 (segment (start 157.48 78.74) (end 157.48 71.12) (width 0.25) (layer "F.Cu") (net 23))
 (segment (start 135.795001 79.915001) (end 138.524999 79.915001) (width 0.25) (layer "F.Cu") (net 23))
 (segment (start 137.16 76.2) (end 152.4 76.2) (width 0.25) (layer "F.Cu") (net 19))
 (segment (start 152.4 76.2) (end 152.4 71.12) (width 0.25) (layer "F.Cu") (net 19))
 (segment (start 144.78 79.18952) (end 159.57048 79.18952) (width 0.25) (layer "F.Cu") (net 1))
 (segment (start 184.245489 80.105489) (end 184.245489 81.575521) (width 0.25) (layer "F.Cu") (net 1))
 (segment (start 137.16 81.28) (end 134.62 81.28) (width 0.25) (layer "F.Cu") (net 1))
 (segment (start 182.88 73.66) (end 180.34 73.66) (width 0.25) (layer "F.Cu") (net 1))
 (segment (start 181.705489 79.226499) (end 182.584479 80.105489) (width 0.25) (layer "F.Cu") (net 1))
 (segment (start 180.34 73.66) (end 181.705489 75.025489) (width 0.25) (layer "F.Cu") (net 1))
 (segment (start 177.8 83.82) (end 172.72 78.74) (width 0.25) (layer "F.Cu") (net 1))
 (segment (start 142.68952 81.28) (end 144.78 79.18952) (width 0.25) (layer "F.Cu") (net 1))
 (segment (start 137.16 81.28) (end 142.68952 81.28) (width 0.25) (layer "F.Cu") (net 1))
 (segment (start 172.72 78.74) (end 160.02 78.74) (width 0.25) (layer "F.Cu") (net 1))
 (segment (start 159.57048 79.18952) (end 160.02 78.74) (width 0.25) (layer "F.Cu") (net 1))
 (segment (start 129.54 81.28) (end 129.54 71.12) (width 0.25) (layer "F.Cu") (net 1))
 (segment (start 182.00101 83.82) (end 177.8 83.82) (width 0.25) (layer "F.Cu") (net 1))
 (segment (start 134.62 81.28) (end 129.54 81.28) (width 0.25) (layer "F.Cu") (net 1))
 (segment (start 181.705489 75.025489) (end 181.705489 79.226499) (width 0.25) (layer "F.Cu") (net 1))
 (segment (start 184.245489 81.575521) (end 182.00101 83.82) (width 0.25) (layer "F.Cu") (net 1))
 (segment (start 182.584479 80.105489) (end 184.245489 80.105489) (width 0.25) (layer "F.Cu") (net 1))
 (segment (start 149.86 86.36) (end 149.86 83.82) (width 0.25) (layer "B.Cu") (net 3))
 (segment (start 149.86 83.82) (end 167.64 83.82) (width 0.25) (layer "B.Cu") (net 3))
 (segment (start 167.64 83.82) (end 167.64 86.36) (width 0.25) (layer "B.Cu") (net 3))
 (segment (start 131.63048 88.45048) (end 131.63048 71.56952) (width 0.25) (layer "B.Cu") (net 3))
 (segment (start 132.08 88.9) (end 131.63048 88.45048) (width 0.25) (layer "B.Cu") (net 3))
 (segment (start 149.86 86.36) (end 147.32 88.9) (width 0.25) (layer "B.Cu") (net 3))
 (segment (start 131.63048 71.56952) (end 132.08 71.12) (width 0.25) (layer "B.Cu") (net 3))
 (segment (start 147.32 88.9) (end 132.08 88.9) (width 0.25) (layer "B.Cu") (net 3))
 (segment (start 145.043322 80.38096) (end 148.494511 76.929771) (width 0.25) (layer "B.Cu") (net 4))
 (segment (start 148.494511 68.093501) (end 147.806499 67.405489) (width 0.25) (layer "B.Cu") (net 4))
 (segment (start 172.456677 80.38096) (end 145.043322 80.38096) (width 0.25) (layer "B.Cu") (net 4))
 (segment (start 142.24 83.184282) (end 142.24 86.36) (width 0.25) (layer "B.Cu") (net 4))
 (segment (start 148.494511 76.929771) (end 148.494511 68.093501) (width 0.25) (layer "B.Cu") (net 4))
 (segment (start 133.254511 67.405489) (end 132.08 68.58) (width 0.25) (layer "B.Cu") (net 4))
 (segment (start 147.806499 67.405489) (end 133.254511 67.405489) (width 0.25) (layer "B.Cu") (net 4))
 (segment (start 175.26 86.36) (end 175.26 83.184283) (width 0.25) (layer "B.Cu") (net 4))
 (segment (start 175.26 83.184283) (end 172.456677 80.38096) (width 0.25) (layer "B.Cu") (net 4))
 (segment (start 145.043322 80.38096) (end 142.24 83.184282) (width 0.25) (layer "B.Cu") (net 4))
 (segment (start 147.32 86.36) (end 145.22952 88.45048) (width 0.25) (layer "B.Cu") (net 5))
 (segment (start 136.71048 88.45048) (end 132.08 83.82) (width 0.25) (layer "B.Cu") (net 5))
 (segment (start 145.22952 88.45048) (end 136.71048 88.45048) (width 0.25) (layer "B.Cu") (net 5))
 (segment (start 170.18 81.28) (end 170.18 86.36) (width 0.25) (layer "B.Cu") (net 5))
 (segment (start 132.08 83.82) (end 132.08 73.66) (width 0.25) (layer "B.Cu") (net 5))
 (segment (start 147.32 81.28) (end 170.18 81.28) (width 0.25) (layer "B.Cu") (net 5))
 (segment (start 132.08 73.66) (end 134.62 71.12) (width 0.25) (layer "B.Cu") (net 5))
 (segment (start 147.32 86.36) (end 147.32 81.28) (width 0.25) (layer "B.Cu") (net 5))
 (segment (start 143.605489 74.834511) (end 135.794511 74.834511) (width 0.25) (layer "F.Cu") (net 13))
 (segment (start 135.794511 74.834511) (end 134.62 73.66) (width 0.25) (layer "F.Cu") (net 13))
 (segment (start 144.78 73.66) (end 143.605489 74.834511) (width 0.25) (layer "F.Cu") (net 13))
 (segment (start 144.78 71.12) (end 144.78 73.66) (width 0.25) (layer "F.Cu") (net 13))
 (segment (start 137.16 73.66) (end 137.16 71.12) (width 0.25) (layer "F.Cu") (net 7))
 (segment (start 181.705489 82.454511) (end 178.974511 82.454511) (width 0.25) (layer "F.Cu") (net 31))
 (segment (start 178.974511 82.454511) (end 167.64 71.12) (width 0.25) (layer "F.Cu") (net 31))
 (segment (start 182.88 81.28) (end 181.705489 82.454511) (width 0.25) (layer "F.Cu") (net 31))
 (segment (start 180.34 81.28) (end 170.18 71.12) (width 0.25) (layer "F.Cu") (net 33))
 (segment (start 162.56 79.18952) (end 162.56 79.4645) (width 0.25) (layer "F.Cu") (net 29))
 (segment (start 162.56 86.36) (end 162.56 79.18952) (width 0.25) (layer "F.Cu") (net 29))
 (via (at 162.56 79.4645) (size 0.8) (drill 0.4) (layers "F.Cu" "B.Cu") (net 29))
 (via (at 162.56 86.36) (size 0.8) (drill 0.4) (layers "F.Cu" "B.Cu") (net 29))
 (segment (start 162.56 73.66) (end 165.1 71.12) (width 0.25) (layer "B.Cu") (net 29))
 (segment (start 160.02 86.36) (end 162.56 86.36) (width 0.25) (layer "B.Cu") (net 29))
 (segment (start 162.56 79.4645) (end 162.56 73.66) (width 0.25) (layer "B.Cu") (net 29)))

